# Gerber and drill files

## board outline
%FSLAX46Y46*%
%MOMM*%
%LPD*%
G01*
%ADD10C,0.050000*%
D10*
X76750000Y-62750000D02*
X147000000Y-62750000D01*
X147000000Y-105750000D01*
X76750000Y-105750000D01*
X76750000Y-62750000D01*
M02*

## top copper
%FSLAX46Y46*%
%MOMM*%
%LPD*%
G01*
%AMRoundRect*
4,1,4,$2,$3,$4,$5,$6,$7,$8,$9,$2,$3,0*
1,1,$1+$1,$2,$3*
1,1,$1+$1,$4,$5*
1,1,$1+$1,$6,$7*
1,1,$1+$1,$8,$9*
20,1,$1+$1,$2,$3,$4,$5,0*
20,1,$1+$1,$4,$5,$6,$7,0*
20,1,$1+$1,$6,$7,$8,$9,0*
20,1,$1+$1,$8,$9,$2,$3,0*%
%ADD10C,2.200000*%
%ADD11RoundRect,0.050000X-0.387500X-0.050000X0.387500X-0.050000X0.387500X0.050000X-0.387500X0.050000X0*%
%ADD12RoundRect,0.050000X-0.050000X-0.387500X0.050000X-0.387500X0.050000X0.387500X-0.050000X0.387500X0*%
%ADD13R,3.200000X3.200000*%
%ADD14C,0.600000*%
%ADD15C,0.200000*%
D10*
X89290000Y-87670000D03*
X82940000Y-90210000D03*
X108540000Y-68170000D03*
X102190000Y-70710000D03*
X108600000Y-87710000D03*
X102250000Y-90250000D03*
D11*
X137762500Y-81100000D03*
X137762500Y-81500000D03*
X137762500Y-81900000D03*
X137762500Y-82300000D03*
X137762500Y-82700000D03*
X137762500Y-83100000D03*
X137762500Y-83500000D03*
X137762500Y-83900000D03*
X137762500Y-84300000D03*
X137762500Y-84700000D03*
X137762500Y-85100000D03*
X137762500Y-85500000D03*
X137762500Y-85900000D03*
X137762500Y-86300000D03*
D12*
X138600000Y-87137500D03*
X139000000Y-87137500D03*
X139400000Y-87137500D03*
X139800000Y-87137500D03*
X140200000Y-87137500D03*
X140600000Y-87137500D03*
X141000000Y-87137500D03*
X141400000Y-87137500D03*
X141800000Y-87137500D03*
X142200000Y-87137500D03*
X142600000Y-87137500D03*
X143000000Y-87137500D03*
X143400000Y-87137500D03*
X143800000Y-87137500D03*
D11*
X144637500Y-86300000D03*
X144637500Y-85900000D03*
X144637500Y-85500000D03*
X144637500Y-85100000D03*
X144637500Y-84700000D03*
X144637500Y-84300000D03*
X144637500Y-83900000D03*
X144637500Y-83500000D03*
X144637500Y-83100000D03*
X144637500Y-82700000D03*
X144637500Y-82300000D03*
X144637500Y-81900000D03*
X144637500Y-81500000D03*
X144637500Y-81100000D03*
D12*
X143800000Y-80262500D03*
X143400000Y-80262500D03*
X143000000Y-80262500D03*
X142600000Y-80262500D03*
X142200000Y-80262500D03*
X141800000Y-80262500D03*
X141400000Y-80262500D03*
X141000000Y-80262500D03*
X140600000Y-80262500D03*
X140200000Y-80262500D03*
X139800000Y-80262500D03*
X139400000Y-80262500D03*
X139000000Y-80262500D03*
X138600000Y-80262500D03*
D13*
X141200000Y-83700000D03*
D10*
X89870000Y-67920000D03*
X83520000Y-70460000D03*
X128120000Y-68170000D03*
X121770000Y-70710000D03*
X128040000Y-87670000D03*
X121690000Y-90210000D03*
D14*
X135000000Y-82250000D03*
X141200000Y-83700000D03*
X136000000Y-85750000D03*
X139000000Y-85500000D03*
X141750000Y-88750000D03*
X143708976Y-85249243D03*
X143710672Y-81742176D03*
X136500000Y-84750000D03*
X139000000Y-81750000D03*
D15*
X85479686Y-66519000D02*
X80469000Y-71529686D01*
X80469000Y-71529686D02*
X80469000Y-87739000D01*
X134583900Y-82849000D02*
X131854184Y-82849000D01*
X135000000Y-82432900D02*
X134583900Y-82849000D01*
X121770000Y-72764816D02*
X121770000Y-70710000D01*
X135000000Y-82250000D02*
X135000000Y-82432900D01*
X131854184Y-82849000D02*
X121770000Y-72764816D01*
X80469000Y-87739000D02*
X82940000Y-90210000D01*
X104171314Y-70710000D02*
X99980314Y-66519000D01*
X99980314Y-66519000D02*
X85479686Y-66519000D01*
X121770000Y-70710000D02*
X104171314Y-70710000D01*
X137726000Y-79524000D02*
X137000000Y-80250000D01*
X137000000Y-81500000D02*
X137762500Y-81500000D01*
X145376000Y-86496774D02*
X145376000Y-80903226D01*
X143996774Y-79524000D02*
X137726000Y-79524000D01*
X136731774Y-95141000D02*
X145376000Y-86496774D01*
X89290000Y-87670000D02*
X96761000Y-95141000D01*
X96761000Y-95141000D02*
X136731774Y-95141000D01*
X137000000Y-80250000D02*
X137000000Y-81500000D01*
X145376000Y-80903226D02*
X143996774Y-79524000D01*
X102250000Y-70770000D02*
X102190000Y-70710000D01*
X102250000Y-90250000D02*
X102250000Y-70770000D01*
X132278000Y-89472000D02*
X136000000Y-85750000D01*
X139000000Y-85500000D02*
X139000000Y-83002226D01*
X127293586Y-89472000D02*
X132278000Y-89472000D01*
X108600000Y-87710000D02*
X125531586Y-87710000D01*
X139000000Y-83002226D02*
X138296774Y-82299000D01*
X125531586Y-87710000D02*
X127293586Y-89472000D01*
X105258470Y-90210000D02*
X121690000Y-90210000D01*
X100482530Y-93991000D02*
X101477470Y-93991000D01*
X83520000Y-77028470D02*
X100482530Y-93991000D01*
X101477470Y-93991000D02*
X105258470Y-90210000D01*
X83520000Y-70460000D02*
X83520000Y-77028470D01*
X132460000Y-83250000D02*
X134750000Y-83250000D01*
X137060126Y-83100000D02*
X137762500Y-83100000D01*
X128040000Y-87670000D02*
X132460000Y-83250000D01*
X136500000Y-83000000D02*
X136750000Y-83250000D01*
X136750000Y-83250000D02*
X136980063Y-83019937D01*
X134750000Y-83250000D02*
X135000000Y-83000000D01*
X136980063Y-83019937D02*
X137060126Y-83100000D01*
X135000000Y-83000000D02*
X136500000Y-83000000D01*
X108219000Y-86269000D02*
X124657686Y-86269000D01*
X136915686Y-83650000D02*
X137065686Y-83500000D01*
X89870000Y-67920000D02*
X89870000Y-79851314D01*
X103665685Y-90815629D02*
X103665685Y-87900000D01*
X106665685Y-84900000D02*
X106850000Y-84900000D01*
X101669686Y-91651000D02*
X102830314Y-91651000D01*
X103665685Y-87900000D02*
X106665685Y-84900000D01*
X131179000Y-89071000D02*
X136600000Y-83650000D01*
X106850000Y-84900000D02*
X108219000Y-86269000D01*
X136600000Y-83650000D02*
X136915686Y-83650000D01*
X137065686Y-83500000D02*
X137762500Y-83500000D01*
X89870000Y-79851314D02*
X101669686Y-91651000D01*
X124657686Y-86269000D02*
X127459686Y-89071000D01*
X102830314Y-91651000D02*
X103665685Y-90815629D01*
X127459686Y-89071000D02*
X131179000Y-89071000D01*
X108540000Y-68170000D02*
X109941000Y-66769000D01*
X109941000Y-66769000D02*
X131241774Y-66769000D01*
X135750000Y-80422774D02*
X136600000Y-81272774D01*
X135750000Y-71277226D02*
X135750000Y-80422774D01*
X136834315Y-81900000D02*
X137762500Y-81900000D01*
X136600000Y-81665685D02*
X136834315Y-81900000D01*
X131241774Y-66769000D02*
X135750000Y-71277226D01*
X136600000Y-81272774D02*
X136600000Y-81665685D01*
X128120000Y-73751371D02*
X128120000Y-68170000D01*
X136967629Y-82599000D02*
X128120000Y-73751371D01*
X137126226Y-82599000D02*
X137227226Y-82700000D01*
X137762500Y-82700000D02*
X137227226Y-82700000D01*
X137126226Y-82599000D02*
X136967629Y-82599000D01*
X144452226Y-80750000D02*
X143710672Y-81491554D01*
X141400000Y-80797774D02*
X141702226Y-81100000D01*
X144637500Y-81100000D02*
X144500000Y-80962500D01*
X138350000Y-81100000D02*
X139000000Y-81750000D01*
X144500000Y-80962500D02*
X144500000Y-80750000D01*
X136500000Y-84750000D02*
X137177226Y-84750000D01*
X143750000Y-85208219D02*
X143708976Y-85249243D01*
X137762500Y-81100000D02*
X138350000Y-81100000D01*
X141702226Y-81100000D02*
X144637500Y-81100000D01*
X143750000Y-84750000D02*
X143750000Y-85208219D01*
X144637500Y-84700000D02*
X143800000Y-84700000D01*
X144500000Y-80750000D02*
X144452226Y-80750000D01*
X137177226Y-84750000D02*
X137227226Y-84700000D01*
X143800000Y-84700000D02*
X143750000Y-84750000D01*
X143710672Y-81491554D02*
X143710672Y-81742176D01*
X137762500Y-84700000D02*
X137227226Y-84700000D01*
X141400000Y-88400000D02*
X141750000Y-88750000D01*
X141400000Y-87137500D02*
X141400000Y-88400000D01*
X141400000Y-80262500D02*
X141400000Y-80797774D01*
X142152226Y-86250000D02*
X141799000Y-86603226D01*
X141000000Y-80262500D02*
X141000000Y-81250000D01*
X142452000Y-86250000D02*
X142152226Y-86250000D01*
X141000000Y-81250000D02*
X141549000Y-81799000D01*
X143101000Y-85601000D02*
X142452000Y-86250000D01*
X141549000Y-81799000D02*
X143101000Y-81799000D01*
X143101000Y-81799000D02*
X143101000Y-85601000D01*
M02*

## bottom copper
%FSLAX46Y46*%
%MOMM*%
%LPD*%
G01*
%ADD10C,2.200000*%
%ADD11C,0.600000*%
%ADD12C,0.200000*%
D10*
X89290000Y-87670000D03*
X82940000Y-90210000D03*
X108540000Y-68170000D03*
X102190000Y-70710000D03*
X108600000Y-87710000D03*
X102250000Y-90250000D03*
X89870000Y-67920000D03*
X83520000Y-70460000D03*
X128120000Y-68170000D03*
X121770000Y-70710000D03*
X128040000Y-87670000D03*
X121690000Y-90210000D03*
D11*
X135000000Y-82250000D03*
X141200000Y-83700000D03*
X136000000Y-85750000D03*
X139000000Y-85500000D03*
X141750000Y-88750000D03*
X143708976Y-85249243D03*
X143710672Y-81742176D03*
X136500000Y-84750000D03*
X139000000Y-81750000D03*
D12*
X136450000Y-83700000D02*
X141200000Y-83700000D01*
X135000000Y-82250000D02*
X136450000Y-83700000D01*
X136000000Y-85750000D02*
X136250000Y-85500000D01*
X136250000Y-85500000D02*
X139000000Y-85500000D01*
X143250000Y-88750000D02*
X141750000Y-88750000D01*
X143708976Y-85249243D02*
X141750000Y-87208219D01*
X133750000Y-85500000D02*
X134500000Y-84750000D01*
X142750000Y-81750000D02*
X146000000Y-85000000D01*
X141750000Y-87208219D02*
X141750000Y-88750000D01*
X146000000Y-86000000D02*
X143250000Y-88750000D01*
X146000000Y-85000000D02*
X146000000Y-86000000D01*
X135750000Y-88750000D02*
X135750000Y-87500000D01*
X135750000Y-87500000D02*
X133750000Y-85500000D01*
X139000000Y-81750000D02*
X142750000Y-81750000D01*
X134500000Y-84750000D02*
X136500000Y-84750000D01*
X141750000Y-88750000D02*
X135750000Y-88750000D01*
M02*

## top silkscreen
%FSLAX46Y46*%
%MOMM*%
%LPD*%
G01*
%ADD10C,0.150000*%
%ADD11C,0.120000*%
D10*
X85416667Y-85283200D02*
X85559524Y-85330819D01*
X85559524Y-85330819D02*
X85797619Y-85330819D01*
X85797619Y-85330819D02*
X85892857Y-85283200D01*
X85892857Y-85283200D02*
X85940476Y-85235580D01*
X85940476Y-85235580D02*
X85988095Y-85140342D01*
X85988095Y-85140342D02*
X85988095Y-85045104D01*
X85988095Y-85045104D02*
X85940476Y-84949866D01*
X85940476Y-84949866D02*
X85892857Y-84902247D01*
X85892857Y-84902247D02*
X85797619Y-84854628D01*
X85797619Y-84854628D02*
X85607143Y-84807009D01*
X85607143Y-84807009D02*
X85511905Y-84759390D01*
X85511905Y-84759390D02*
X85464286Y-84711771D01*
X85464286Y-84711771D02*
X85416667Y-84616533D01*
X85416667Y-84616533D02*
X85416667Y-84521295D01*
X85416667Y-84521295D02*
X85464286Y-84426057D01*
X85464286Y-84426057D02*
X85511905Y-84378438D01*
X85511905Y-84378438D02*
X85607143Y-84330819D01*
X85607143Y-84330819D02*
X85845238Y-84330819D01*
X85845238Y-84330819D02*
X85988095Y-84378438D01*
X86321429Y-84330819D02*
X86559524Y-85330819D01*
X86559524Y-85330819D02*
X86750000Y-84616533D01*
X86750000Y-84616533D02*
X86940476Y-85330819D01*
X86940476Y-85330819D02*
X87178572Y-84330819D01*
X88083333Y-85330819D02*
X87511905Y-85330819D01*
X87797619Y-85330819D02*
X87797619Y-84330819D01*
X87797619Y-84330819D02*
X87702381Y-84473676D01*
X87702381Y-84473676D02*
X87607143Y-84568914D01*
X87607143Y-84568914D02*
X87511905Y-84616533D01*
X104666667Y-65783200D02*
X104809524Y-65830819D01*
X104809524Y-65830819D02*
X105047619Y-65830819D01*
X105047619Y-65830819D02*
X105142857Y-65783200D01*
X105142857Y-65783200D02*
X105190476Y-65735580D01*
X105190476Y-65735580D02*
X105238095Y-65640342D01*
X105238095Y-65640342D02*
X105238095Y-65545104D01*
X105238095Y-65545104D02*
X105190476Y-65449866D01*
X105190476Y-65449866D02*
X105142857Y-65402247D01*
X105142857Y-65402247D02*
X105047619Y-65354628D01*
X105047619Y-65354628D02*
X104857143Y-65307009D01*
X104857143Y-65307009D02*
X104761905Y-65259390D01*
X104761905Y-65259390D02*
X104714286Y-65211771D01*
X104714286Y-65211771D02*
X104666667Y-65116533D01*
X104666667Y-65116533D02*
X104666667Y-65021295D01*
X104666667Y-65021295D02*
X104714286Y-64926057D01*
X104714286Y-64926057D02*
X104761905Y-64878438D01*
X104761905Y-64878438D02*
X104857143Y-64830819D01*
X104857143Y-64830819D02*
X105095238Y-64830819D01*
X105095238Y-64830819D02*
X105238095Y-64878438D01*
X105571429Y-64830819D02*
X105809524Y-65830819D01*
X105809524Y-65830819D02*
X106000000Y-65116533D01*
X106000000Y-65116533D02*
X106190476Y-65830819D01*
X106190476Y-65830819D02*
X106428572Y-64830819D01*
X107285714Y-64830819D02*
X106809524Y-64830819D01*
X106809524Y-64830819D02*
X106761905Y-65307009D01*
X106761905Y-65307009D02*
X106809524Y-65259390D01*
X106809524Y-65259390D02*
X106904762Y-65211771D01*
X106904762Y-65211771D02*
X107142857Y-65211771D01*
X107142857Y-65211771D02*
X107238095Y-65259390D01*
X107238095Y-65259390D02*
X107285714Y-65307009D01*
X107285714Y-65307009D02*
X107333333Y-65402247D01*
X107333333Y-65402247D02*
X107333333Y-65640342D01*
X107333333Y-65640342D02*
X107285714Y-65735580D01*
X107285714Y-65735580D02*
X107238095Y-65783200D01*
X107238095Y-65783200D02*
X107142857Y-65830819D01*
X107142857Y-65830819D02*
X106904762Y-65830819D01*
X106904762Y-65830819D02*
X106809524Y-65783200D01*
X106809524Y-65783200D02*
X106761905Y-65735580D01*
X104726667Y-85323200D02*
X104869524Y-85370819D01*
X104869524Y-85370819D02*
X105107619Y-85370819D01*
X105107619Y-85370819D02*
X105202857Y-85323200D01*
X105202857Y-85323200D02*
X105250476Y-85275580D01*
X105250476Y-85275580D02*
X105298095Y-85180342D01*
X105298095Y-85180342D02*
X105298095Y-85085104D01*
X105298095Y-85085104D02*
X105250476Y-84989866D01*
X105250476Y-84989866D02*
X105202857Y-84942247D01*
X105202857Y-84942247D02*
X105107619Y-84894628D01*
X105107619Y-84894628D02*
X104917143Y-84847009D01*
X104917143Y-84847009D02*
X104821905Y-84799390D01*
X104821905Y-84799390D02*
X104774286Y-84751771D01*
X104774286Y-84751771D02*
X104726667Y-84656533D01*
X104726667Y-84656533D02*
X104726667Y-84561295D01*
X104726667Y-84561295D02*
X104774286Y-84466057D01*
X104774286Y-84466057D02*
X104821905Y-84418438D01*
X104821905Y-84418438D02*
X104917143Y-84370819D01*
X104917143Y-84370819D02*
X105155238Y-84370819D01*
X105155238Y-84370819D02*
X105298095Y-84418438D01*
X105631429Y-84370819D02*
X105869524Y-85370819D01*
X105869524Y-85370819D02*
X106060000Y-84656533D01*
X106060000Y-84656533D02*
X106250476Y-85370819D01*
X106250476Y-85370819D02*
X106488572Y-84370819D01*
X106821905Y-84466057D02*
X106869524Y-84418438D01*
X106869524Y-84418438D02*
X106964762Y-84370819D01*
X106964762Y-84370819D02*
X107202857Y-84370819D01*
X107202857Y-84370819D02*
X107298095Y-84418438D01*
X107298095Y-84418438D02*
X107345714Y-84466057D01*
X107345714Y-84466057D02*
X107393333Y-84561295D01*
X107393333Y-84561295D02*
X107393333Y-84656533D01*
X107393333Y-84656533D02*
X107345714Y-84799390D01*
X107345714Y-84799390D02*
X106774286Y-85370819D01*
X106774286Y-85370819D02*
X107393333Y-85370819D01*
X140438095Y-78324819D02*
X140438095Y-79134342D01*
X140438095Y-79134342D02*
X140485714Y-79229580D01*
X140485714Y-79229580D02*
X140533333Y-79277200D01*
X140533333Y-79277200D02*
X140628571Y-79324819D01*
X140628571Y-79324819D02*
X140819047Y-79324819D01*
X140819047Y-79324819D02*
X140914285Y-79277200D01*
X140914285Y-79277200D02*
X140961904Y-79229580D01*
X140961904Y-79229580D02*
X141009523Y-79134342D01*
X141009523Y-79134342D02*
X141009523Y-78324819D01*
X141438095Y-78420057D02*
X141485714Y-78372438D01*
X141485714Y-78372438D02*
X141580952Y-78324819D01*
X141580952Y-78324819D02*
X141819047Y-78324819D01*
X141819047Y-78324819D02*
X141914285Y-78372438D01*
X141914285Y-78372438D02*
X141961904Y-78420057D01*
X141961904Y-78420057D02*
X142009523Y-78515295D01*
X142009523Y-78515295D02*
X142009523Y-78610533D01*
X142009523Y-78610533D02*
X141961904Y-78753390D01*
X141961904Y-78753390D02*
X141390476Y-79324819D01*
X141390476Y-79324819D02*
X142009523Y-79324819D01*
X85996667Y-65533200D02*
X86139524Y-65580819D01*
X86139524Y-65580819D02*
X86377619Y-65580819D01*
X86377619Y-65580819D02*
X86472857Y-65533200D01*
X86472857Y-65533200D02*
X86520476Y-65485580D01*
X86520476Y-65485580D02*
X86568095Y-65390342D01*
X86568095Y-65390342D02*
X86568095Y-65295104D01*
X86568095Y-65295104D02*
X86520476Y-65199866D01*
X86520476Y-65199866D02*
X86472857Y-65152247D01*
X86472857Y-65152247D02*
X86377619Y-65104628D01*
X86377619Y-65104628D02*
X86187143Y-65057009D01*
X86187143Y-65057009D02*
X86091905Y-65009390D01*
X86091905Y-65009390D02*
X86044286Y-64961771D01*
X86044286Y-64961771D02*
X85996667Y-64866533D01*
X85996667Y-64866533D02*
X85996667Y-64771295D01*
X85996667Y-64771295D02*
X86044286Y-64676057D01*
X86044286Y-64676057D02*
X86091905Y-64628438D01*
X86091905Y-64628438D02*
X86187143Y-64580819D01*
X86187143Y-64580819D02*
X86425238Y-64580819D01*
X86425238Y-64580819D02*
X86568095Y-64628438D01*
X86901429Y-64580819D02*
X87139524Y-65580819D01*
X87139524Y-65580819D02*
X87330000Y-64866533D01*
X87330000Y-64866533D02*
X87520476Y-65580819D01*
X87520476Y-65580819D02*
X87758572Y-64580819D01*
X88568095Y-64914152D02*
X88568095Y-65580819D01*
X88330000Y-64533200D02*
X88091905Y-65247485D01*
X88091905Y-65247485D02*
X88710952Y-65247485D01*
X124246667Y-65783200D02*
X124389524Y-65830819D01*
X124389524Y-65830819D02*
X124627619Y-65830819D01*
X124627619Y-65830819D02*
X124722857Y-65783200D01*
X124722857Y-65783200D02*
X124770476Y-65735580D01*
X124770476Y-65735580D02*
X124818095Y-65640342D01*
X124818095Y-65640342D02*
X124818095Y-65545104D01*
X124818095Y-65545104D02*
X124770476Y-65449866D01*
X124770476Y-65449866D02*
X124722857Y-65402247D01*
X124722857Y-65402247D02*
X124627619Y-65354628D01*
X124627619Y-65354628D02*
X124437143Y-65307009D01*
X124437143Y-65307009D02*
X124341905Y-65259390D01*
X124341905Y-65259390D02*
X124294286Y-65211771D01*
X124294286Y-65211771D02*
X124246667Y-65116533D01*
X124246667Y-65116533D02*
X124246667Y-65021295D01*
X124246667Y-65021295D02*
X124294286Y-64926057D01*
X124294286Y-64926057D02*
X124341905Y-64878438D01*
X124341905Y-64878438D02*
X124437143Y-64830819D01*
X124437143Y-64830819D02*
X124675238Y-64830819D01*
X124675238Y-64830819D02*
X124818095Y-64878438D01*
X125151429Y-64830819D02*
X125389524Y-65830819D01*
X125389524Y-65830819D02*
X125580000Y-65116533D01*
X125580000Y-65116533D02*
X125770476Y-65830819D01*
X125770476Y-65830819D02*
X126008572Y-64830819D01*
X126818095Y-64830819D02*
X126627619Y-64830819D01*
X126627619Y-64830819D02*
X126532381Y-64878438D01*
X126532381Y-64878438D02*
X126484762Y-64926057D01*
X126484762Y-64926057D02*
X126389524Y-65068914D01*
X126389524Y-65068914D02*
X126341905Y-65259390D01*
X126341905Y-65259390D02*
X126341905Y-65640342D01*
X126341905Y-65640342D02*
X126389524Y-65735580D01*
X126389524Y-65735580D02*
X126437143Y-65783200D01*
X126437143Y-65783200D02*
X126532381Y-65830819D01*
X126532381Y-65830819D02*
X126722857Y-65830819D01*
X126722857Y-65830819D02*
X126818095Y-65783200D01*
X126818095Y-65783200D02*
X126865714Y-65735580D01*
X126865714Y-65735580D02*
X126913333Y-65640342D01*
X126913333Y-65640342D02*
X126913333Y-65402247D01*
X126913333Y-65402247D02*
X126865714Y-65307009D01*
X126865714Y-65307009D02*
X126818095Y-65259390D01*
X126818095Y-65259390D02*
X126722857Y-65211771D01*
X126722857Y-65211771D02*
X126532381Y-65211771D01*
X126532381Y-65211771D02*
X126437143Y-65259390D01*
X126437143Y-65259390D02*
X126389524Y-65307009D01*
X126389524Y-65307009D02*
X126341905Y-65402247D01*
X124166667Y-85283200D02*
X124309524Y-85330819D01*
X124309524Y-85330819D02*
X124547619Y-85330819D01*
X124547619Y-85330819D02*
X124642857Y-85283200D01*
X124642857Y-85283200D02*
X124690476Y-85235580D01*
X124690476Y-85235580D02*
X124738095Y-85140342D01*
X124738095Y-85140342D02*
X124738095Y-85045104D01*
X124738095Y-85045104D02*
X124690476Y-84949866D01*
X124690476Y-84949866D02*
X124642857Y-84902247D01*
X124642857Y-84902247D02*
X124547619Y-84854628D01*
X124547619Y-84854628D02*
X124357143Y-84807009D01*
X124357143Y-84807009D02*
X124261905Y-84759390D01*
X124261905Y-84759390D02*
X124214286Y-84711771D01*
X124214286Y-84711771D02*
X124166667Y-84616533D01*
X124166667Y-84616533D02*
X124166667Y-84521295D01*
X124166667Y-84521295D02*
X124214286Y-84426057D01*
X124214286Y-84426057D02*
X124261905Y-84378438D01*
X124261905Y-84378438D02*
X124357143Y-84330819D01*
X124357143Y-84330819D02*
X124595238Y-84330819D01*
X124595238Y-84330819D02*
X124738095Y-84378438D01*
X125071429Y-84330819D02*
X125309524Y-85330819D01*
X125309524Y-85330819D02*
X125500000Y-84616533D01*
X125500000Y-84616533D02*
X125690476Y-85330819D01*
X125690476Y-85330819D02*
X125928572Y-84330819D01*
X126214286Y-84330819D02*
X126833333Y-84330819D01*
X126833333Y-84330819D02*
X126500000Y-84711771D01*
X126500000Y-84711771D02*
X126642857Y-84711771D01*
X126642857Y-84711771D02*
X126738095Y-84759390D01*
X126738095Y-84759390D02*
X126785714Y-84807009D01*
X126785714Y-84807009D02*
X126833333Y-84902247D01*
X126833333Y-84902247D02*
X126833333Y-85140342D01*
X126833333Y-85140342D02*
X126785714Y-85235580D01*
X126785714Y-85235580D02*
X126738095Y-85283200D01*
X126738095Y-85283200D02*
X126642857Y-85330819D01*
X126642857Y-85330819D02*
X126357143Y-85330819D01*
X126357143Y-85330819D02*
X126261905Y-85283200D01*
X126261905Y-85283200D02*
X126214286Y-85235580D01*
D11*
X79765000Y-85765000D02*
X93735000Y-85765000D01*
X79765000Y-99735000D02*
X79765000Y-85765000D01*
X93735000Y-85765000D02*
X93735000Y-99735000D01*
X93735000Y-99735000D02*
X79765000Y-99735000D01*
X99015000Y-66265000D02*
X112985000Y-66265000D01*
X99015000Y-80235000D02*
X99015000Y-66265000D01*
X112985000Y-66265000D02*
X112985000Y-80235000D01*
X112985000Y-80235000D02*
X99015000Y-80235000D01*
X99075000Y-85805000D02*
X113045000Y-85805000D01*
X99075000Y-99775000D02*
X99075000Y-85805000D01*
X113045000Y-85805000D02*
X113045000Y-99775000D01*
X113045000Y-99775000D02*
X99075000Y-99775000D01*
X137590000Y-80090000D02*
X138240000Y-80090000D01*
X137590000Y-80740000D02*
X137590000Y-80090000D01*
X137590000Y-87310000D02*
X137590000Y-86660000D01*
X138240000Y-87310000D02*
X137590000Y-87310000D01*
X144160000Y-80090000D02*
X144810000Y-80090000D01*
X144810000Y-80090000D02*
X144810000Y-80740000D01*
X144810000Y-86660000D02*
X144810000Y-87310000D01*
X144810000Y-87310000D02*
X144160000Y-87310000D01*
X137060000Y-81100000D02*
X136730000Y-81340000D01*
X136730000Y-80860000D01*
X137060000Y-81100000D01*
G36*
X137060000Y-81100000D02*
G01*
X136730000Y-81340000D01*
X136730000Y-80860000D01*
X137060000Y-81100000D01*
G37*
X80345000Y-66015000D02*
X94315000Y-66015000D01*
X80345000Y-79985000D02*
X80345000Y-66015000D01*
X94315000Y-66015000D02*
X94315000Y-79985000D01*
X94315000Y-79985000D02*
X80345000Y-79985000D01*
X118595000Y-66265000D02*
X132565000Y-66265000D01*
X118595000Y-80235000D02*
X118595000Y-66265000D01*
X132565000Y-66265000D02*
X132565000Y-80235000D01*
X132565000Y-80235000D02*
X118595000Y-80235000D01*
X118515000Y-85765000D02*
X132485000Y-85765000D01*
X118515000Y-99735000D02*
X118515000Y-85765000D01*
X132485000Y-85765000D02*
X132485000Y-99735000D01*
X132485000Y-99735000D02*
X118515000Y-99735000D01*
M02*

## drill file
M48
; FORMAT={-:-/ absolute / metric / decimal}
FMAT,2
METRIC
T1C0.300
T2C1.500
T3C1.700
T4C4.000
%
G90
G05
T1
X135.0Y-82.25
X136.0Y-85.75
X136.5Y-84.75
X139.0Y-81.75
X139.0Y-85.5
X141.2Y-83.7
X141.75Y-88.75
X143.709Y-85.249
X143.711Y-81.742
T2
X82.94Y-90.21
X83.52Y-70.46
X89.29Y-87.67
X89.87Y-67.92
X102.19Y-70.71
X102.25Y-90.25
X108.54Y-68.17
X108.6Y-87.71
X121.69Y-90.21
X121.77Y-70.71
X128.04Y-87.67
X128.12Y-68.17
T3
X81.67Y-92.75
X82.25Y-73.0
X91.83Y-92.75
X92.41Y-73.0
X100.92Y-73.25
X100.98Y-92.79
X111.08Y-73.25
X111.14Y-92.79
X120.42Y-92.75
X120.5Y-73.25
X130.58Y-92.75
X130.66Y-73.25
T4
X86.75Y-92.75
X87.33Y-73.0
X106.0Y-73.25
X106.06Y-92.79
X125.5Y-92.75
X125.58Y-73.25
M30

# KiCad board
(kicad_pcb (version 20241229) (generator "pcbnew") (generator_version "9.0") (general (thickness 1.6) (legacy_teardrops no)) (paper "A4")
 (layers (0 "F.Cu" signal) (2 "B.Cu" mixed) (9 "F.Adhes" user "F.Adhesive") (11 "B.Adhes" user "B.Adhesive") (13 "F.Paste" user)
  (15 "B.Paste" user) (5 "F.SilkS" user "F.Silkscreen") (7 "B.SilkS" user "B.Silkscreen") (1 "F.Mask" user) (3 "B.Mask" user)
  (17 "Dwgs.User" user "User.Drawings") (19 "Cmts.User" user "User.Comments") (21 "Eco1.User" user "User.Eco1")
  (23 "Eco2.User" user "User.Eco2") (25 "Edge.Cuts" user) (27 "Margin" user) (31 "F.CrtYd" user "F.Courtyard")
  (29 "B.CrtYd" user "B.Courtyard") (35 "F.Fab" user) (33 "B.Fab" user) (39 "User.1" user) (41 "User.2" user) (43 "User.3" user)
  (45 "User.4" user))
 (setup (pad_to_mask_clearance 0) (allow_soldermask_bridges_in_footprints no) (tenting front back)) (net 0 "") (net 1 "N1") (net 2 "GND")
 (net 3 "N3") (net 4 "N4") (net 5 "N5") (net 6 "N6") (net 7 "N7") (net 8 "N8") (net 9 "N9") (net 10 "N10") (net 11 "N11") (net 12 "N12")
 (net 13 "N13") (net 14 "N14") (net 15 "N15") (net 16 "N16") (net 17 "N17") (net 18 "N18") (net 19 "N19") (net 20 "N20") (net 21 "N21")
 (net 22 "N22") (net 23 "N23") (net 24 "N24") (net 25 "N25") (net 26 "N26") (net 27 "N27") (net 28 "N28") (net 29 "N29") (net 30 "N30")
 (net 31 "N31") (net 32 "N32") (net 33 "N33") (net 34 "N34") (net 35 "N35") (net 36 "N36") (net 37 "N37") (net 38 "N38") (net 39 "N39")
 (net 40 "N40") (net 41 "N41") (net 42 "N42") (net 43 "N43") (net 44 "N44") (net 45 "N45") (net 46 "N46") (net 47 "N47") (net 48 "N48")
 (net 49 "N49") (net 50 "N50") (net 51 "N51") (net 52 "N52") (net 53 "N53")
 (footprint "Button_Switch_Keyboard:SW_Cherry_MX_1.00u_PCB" (layer "F.Cu") (at 89.29 87.67)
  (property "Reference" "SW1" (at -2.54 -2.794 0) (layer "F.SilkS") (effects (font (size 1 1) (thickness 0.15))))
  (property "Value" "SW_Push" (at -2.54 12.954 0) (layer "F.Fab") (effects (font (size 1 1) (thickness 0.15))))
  (fp_line (start -9.525 -1.905) (end 4.445 -1.905) (stroke (width 0.12) (type solid)) (layer "F.SilkS"))
  (fp_line (start -9.525 12.065) (end -9.525 -1.905) (stroke (width 0.12) (type solid)) (layer "F.SilkS"))
  (fp_line (start 4.445 -1.905) (end 4.445 12.065) (stroke (width 0.12) (type solid)) (layer "F.SilkS"))
  (fp_line (start 4.445 12.065) (end -9.525 12.065) (stroke (width 0.12) (type solid)) (layer "F.SilkS"))
  (pad "" np_thru_hole circle (at -7.62 5.08) (size 1.7 1.7) (drill 1.7) (layers "*.Cu" "*.Mask"))
  (pad "" np_thru_hole circle (at -2.54 5.08) (size 4 4) (drill 4) (layers "*.Cu" "*.Mask"))
  (pad "" np_thru_hole circle (at 2.54 5.08) (size 1.7 1.7) (drill 1.7) (layers "*.Cu" "*.Mask"))
  (pad "1" thru_hole circle (at 0 0) (size 2.2 2.2) (drill 1.5) (layers "*.Cu" "*.Mask") (remove_unused_layers no) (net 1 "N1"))
  (pad "2" thru_hole circle (at -6.35 2.54) (size 2.2 2.2) (drill 1.5) (layers "*.Cu" "*.Mask") (remove_unused_layers no) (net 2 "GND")))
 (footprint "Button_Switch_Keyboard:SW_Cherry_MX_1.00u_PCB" (layer "F.Cu") (at 108.54 68.17)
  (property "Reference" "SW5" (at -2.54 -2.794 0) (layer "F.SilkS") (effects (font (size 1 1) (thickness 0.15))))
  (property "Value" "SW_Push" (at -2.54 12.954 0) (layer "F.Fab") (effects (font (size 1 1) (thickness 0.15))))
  (fp_line (start -9.525 -1.905) (end 4.445 -1.905) (stroke (width 0.12) (type solid)) (layer "F.SilkS"))
  (fp_line (start -9.525 12.065) (end -9.525 -1.905) (stroke (width 0.12) (type solid)) (layer "F.SilkS"))
  (fp_line (start 4.445 -1.905) (end 4.445 12.065) (stroke (width 0.12) (type solid)) (layer "F.SilkS"))
  (fp_line (start 4.445 12.065) (end -9.525 12.065) (stroke (width 0.12) (type solid)) (layer "F.SilkS"))
  (pad "" np_thru_hole circle (at -7.62 5.08) (size 1.7 1.7) (drill 1.7) (layers "*.Cu" "*.Mask"))
  (pad "" np_thru_hole circle (at -2.54 5.08) (size 4 4) (drill 4) (layers "*.Cu" "*.Mask"))
  (pad "" np_thru_hole circle (at 2.54 5.08) (size 1.7 1.7) (drill 1.7) (layers "*.Cu" "*.Mask"))
  (pad "1" thru_hole circle (at 0 0) (size 2.2 2.2) (drill 1.5) (layers "*.Cu" "*.Mask") (remove_unused_layers no) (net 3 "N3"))
  (pad "2" thru_hole circle (at -6.35 2.54) (size 2.2 2.2) (drill 1.5) (layers "*.Cu" "*.Mask") (remove_unused_layers no) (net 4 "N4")))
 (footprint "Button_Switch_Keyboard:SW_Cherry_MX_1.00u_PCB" (layer "F.Cu") (at 108.6 87.71)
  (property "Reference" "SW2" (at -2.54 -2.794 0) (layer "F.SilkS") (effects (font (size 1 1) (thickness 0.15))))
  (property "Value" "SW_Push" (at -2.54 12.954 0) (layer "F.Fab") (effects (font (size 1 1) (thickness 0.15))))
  (fp_line (start -9.525 -1.905) (end 4.445 -1.905) (stroke (width 0.12) (type solid)) (layer "F.SilkS"))
  (fp_line (start -9.525 12.065) (end -9.525 -1.905) (stroke (width 0.12) (type solid)) (layer "F.SilkS"))
  (fp_line (start 4.445 -1.905) (end 4.445 12.065) (stroke (width 0.12) (type solid)) (layer "F.SilkS"))
  (fp_line (start 4.445 12.065) (end -9.525 12.065) (stroke (width 0.12) (type solid)) (layer "F.SilkS"))
  (pad "" np_thru_hole circle (at -7.62 5.08) (size 1.7 1.7) (drill 1.7) (layers "*.Cu" "*.Mask"))
  (pad "" np_thru_hole circle (at -2.54 5.08) (size 4 4) (drill 4) (layers "*.Cu" "*.Mask"))
  (pad "" np_thru_hole circle (at 2.54 5.08) (size 1.7 1.7) (drill 1.7) (layers "*.Cu" "*.Mask"))
  (pad "1" thru_hole circle (at 0 0) (size 2.2 2.2) (drill 1.5) (layers "*.Cu" "*.Mask") (remove_unused_layers no) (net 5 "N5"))
  (pad "2" thru_hole circle (at -6.35 2.54) (size 2.2 2.2) (drill 1.5) (layers "*.Cu" "*.Mask") (remove_unused_layers no) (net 4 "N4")))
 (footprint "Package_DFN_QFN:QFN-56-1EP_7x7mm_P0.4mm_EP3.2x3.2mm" (layer "F.Cu") (at 141.2 83.7)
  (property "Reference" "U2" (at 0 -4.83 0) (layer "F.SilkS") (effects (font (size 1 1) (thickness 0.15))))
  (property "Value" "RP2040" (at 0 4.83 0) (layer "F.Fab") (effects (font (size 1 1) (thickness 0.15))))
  (fp_line (start -3.61 -3.61) (end -2.96 -3.61) (stroke (width 0.12) (type solid)) (layer "F.SilkS"))
  (fp_line (start -3.61 -2.96) (end -3.61 -3.61) (stroke (width 0.12) (type solid)) (layer "F.SilkS"))
  (fp_line (start -3.61 3.61) (end -3.61 2.96) (stroke (width 0.12) (type solid)) (layer "F.SilkS"))
  (fp_line (start -2.96 3.61) (end -3.61 3.61) (stroke (width 0.12) (type solid)) (layer "F.SilkS"))
  (fp_line (start 2.96 -3.61) (end 3.61 -3.61) (stroke (width 0.12) (type solid)) (layer "F.SilkS"))
  (fp_line (start 3.61 -3.61) (end 3.61 -2.96) (stroke (width 0.12) (type solid)) (layer "F.SilkS"))
  (fp_line (start 3.61 2.96) (end 3.61 3.61) (stroke (width 0.12) (type solid)) (layer "F.SilkS"))
  (fp_line (start 3.61 3.61) (end 2.96 3.61) (stroke (width 0.12) (type solid)) (layer "F.SilkS"))
  (fp_poly (pts (xy -4.14 -2.6) (xy -4.47 -2.36) (xy -4.47 -2.84)) (stroke (width 0.12) (type solid)) (fill yes) (layer "F.SilkS"))
  (pad "" smd roundrect (at -0.8 -0.8) (size 1.29 1.29) (layers "F.Paste") (roundrect_rratio 0.193798))
  (pad "" smd roundrect (at -0.8 0.8) (size 1.29 1.29) (layers "F.Paste") (roundrect_rratio 0.193798))
  (pad "" smd roundrect (at 0.8 -0.8) (size 1.29 1.29) (layers "F.Paste") (roundrect_rratio 0.193798))
  (pad "" smd roundrect (at 0.8 0.8) (size 1.29 1.29) (layers "F.Paste") (roundrect_rratio 0.193798))
  (pad "1" smd roundrect (at -3.4375 -2.6) (size 0.875 0.2) (layers "F.Cu" "F.Mask" "F.Paste") (roundrect_rratio 0.25) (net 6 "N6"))
  (pad "2" smd roundrect (at -3.4375 -2.2) (size 0.875 0.2) (layers "F.Cu" "F.Mask" "F.Paste") (roundrect_rratio 0.25) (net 1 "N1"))
  (pad "3" smd roundrect (at -3.4375 -1.8) (size 0.875 0.2) (layers "F.Cu" "F.Mask" "F.Paste") (roundrect_rratio 0.25) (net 3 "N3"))
  (pad "4" smd roundrect (at -3.4375 -1.4) (size 0.875 0.2) (layers "F.Cu" "F.Mask" "F.Paste") (roundrect_rratio 0.25) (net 5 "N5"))
  (pad "5" smd roundrect (at -3.4375 -1) (size 0.875 0.2) (layers "F.Cu" "F.Mask" "F.Paste") (roundrect_rratio 0.25) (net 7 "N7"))
  (pad "6" smd roundrect (at -3.4375 -0.6) (size 0.875 0.2) (layers "F.Cu" "F.Mask" "F.Paste") (roundrect_rratio 0.25) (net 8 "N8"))
  (pad "7" smd roundrect (at -3.4375 -0.2) (size 0.875 0.2) (layers "F.Cu" "F.Mask" "F.Paste") (roundrect_rratio 0.25) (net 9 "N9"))
  (pad "8" smd roundrect (at -3.4375 0.2) (size 0.875 0.2) (layers "F.Cu" "F.Mask" "F.Paste") (roundrect_rratio 0.25) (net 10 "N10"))
  (pad "9" smd roundrect (at -3.4375 0.6) (size 0.875 0.2) (layers "F.Cu" "F.Mask" "F.Paste") (roundrect_rratio 0.25) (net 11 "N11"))
  (pad "10" smd roundrect (at -3.4375 1) (size 0.875 0.2) (layers "F.Cu" "F.Mask" "F.Paste") (roundrect_rratio 0.25) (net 6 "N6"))
  (pad "11" smd roundrect (at -3.4375 1.4) (size 0.875 0.2) (layers "F.Cu" "F.Mask" "F.Paste") (roundrect_rratio 0.25) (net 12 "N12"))
  (pad "12" smd roundrect (at -3.4375 1.8) (size 0.875 0.2) (layers "F.Cu" "F.Mask" "F.Paste") (roundrect_rratio 0.25) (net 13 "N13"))
  (pad "13" smd roundrect (at -3.4375 2.2) (size 0.875 0.2) (layers "F.Cu" "F.Mask" "F.Paste") (roundrect_rratio 0.25) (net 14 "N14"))
  (pad "14" smd roundrect (at -3.4375 2.6) (size 0.875 0.2) (layers "F.Cu" "F.Mask" "F.Paste") (roundrect_rratio 0.25) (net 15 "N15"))
  (pad "15" smd roundrect (at -2.6 3.4375) (size 0.2 0.875) (layers "F.Cu" "F.Mask" "F.Paste") (roundrect_rratio 0.25) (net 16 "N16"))
  (pad "16" smd roundrect (at -2.2 3.4375) (size 0.2 0.875) (layers "F.Cu" "F.Mask" "F.Paste") (roundrect_rratio 0.25) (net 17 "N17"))
  (pad "17" smd roundrect (at -1.8 3.4375) (size 0.2 0.875) (layers "F.Cu" "F.Mask" "F.Paste") (roundrect_rratio 0.25) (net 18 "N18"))
  (pad "18" smd roundrect (at -1.4 3.4375) (size 0.2 0.875) (layers "F.Cu" "F.Mask" "F.Paste") (roundrect_rratio 0.25) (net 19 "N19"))
  (pad "19" smd roundrect (at -1 3.4375) (size 0.2 0.875) (layers "F.Cu" "F.Mask" "F.Paste") (roundrect_rratio 0.25) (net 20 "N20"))
  (pad "20" smd roundrect (at -0.6 3.4375) (size 0.2 0.875) (layers "F.Cu" "F.Mask" "F.Paste") (roundrect_rratio 0.25) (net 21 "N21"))
  (pad "21" smd roundrect (at -0.2 3.4375) (size 0.2 0.875) (layers "F.Cu" "F.Mask" "F.Paste") (roundrect_rratio 0.25) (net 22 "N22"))
  (pad "22" smd roundrect (at 0.2 3.4375) (size 0.2 0.875) (layers "F.Cu" "F.Mask" "F.Paste") (roundrect_rratio 0.25) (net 6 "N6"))
  (pad "23" smd roundrect (at 0.6 3.4375) (size 0.2 0.875) (layers "F.Cu" "F.Mask" "F.Paste") (roundrect_rratio 0.25) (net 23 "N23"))
  (pad "24" smd roundrect (at 1 3.4375) (size 0.2 0.875) (layers "F.Cu" "F.Mask" "F.Paste") (roundrect_rratio 0.25) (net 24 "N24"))
  (pad "25" smd roundrect (at 1.4 3.4375) (size 0.2 0.875) (layers "F.Cu" "F.Mask" "F.Paste") (roundrect_rratio 0.25) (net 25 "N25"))
  (pad "26" smd roundrect (at 1.8 3.4375) (size 0.2 0.875) (layers "F.Cu" "F.Mask" "F.Paste") (roundrect_rratio 0.25) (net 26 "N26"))
  (pad "27" smd roundrect (at 2.2 3.4375) (size 0.2 0.875) (layers "F.Cu" "F.Mask" "F.Paste") (roundrect_rratio 0.25) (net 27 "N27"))
  (pad "28" smd roundrect (at 2.6 3.4375) (size 0.2 0.875) (layers "F.Cu" "F.Mask" "F.Paste") (roundrect_rratio 0.25) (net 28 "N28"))
  (pad "29" smd roundrect (at 3.4375 2.6) (size 0.875 0.2) (layers "F.Cu" "F.Mask" "F.Paste") (roundrect_rratio 0.25) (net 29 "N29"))
  (pad "30" smd roundrect (at 3.4375 2.2) (size 0.875 0.2) (layers "F.Cu" "F.Mask" "F.Paste") (roundrect_rratio 0.25) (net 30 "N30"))
  (pad "31" smd roundrect (at 3.4375 1.8) (size 0.875 0.2) (layers "F.Cu" "F.Mask" "F.Paste") (roundrect_rratio 0.25) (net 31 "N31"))
  (pad "32" smd roundrect (at 3.4375 1.4) (size 0.875 0.2) (layers "F.Cu" "F.Mask" "F.Paste") (roundrect_rratio 0.25) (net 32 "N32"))
  (pad "33" smd roundrect (at 3.4375 1) (size 0.875 0.2) (layers "F.Cu" "F.Mask" "F.Paste") (roundrect_rratio 0.25) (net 6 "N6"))
  (pad "34" smd roundrect (at 3.4375 0.6) (size 0.875 0.2) (layers "F.Cu" "F.Mask" "F.Paste") (roundrect_rratio 0.25) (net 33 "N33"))
  (pad "35" smd roundrect (at 3.4375 0.2) (size 0.875 0.2) (layers "F.Cu" "F.Mask" "F.Paste") (roundrect_rratio 0.25) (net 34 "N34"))
  (pad "36" smd roundrect (at 3.4375 -0.2) (size 0.875 0.2) (layers "F.Cu" "F.Mask" "F.Paste") (roundrect_rratio 0.25) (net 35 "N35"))
  (pad "37" smd roundrect (at 3.4375 -0.6) (size 0.875 0.2) (layers "F.Cu" "F.Mask" "F.Paste") (roundrect_rratio 0.25) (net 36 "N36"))
  (pad "38" smd roundrect (at 3.4375 -1) (size 0.875 0.2) (layers "F.Cu" "F.Mask" "F.Paste") (roundrect_rratio 0.25) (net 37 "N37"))
  (pad "39" smd roundrect (at 3.4375 -1.4) (size 0.875 0.2) (layers "F.Cu" "F.Mask" "F.Paste") (roundrect_rratio 0.25) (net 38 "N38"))
  (pad "40" smd roundrect (at 3.4375 -1.8) (size 0.875 0.2) (layers "F.Cu" "F.Mask" "F.Paste") (roundrect_rratio 0.25) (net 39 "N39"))
  (pad "41" smd roundrect (at 3.4375 -2.2) (size 0.875 0.2) (layers "F.Cu" "F.Mask" "F.Paste") (roundrect_rratio 0.25) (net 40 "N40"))
  (pad "42" smd roundrect (at 3.4375 -2.6) (size 0.875 0.2) (layers "F.Cu" "F.Mask" "F.Paste") (roundrect_rratio 0.25) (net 6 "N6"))
  (pad "43" smd roundrect (at 2.6 -3.4375) (size 0.2 0.875) (layers "F.Cu" "F.Mask" "F.Paste") (roundrect_rratio 0.25) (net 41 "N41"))
  (pad "44" smd roundrect (at 2.2 -3.4375) (size 0.2 0.875) (layers "F.Cu" "F.Mask" "F.Paste") (roundrect_rratio 0.25) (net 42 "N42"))
  (pad "45" smd roundrect (at 1.8 -3.4375) (size 0.2 0.875) (layers "F.Cu" "F.Mask" "F.Paste") (roundrect_rratio 0.25) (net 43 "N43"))
  (pad "46" smd roundrect (at 1.4 -3.4375) (size 0.2 0.875) (layers "F.Cu" "F.Mask" "F.Paste") (roundrect_rratio 0.25) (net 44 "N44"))
  (pad "47" smd roundrect (at 1 -3.4375) (size 0.2 0.875) (layers "F.Cu" "F.Mask" "F.Paste") (roundrect_rratio 0.25) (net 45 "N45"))
  (pad "48" smd roundrect (at 0.6 -3.4375) (size 0.2 0.875) (layers "F.Cu" "F.Mask" "F.Paste") (roundrect_rratio 0.25) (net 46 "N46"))
  (pad "49" smd roundrect (at 0.2 -3.4375) (size 0.2 0.875) (layers "F.Cu" "F.Mask" "F.Paste") (roundrect_rratio 0.25) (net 6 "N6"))
  (pad "50" smd roundrect (at -0.2 -3.4375) (size 0.2 0.875) (layers "F.Cu" "F.Mask" "F.Paste") (roundrect_rratio 0.25) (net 23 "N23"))
  (pad "51" smd roundrect (at -0.6 -3.4375) (size 0.2 0.875) (layers "F.Cu" "F.Mask" "F.Paste") (roundrect_rratio 0.25) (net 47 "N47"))
  (pad "52" smd roundrect (at -1 -3.4375) (size 0.2 0.875) (layers "F.Cu" "F.Mask" "F.Paste") (roundrect_rratio 0.25) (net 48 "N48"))
  (pad "53" smd roundrect (at -1.4 -3.4375) (size 0.2 0.875) (layers "F.Cu" "F.Mask" "F.Paste") (roundrect_rratio 0.25) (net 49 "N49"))
  (pad "54" smd roundrect (at -1.8 -3.4375) (size 0.2 0.875) (layers "F.Cu" "F.Mask" "F.Paste") (roundrect_rratio 0.25) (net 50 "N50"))
  (pad "55" smd roundrect (at -2.2 -3.4375) (size 0.2 0.875) (layers "F.Cu" "F.Mask" "F.Paste") (roundrect_rratio 0.25) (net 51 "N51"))
  (pad "56" smd roundrect (at -2.6 -3.4375) (size 0.2 0.875) (layers "F.Cu" "F.Mask" "F.Paste") (roundrect_rratio 0.25) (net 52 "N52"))
  (pad "57" smd rect (at 0 0) (size 3.2 3.2) (layers "F.Cu" "F.Mask") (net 2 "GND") (zone_connect 2)))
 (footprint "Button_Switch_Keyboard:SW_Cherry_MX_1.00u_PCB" (layer "F.Cu") (at 89.87 67.92)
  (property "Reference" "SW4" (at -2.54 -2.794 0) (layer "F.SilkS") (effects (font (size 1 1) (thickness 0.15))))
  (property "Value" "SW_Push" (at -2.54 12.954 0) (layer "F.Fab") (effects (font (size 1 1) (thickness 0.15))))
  (fp_line (start -9.525 -1.905) (end 4.445 -1.905) (stroke (width 0.12) (type solid)) (layer "F.SilkS"))
  (fp_line (start -9.525 12.065) (end -9.525 -1.905) (stroke (width 0.12) (type solid)) (layer "F.SilkS"))
  (fp_line (start 4.445 -1.905) (end 4.445 12.065) (stroke (width 0.12) (type solid)) (layer "F.SilkS"))
  (fp_line (start 4.445 12.065) (end -9.525 12.065) (stroke (width 0.12) (type solid)) (layer "F.SilkS"))
  (pad "" np_thru_hole circle (at -7.62 5.08) (size 1.7 1.7) (drill 1.7) (layers "*.Cu" "*.Mask"))
  (pad "" np_thru_hole circle (at -2.54 5.08) (size 4 4) (drill 4) (layers "*.Cu" "*.Mask"))
  (pad "" np_thru_hole circle (at 2.54 5.08) (size 1.7 1.7) (drill 1.7) (layers "*.Cu" "*.Mask"))
  (pad "1" thru_hole circle (at 0 0) (size 2.2 2.2) (drill 1.5) (layers "*.Cu" "*.Mask") (remove_unused_layers no) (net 9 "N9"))
  (pad "2" thru_hole circle (at -6.35 2.54) (size 2.2 2.2) (drill 1.5) (layers "*.Cu" "*.Mask") (remove_unused_layers no) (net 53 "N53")))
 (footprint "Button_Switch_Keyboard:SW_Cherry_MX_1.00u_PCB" (layer "F.Cu") (at 128.12 68.17)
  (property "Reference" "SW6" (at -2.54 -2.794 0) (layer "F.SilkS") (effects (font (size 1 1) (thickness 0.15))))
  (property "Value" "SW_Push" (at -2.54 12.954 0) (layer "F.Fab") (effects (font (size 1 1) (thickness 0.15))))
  (fp_line (start -9.525 -1.905) (end 4.445 -1.905) (stroke (width 0.12) (type solid)) (layer "F.SilkS"))
  (fp_line (start -9.525 12.065) (end -9.525 -1.905) (stroke (width 0.12) (type solid)) (layer "F.SilkS"))
  (fp_line (start 4.445 -1.905) (end 4.445 12.065) (stroke (width 0.12) (type solid)) (layer "F.SilkS"))
  (fp_line (start 4.445 12.065) (end -9.525 12.065) (stroke (width 0.12) (type solid)) (layer "F.SilkS"))
  (pad "" np_thru_hole circle (at -7.62 5.08) (size 1.7 1.7) (drill 1.7) (layers "*.Cu" "*.Mask"))
  (pad "" np_thru_hole circle (at -2.54 5.08) (size 4 4) (drill 4) (layers "*.Cu" "*.Mask"))
  (pad "" np_thru_hole circle (at 2.54 5.08) (size 1.7 1.7) (drill 1.7) (layers "*.Cu" "*.Mask"))
  (pad "1" thru_hole circle (at 0 0) (size 2.2 2.2) (drill 1.5) (layers "*.Cu" "*.Mask") (remove_unused_layers no) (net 7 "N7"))
  (pad "2" thru_hole circle (at -6.35 2.54) (size 2.2 2.2) (drill 1.5) (layers "*.Cu" "*.Mask") (remove_unused_layers no) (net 2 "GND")))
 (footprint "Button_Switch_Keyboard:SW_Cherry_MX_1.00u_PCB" (layer "F.Cu") (at 128.04 87.67)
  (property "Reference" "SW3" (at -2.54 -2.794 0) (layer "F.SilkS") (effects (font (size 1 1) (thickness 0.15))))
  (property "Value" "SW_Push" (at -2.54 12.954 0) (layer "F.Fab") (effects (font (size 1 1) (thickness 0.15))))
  (fp_line (start -9.525 -1.905) (end 4.445 -1.905) (stroke (width 0.12) (type solid)) (layer "F.SilkS"))
  (fp_line (start -9.525 12.065) (end -9.525 -1.905) (stroke (width 0.12) (type solid)) (layer "F.SilkS"))
  (fp_line (start 4.445 -1.905) (end 4.445 12.065) (stroke (width 0.12) (type solid)) (layer "F.SilkS"))
  (fp_line (start 4.445 12.065) (end -9.525 12.065) (stroke (width 0.12) (type solid)) (layer "F.SilkS"))
  (pad "" np_thru_hole circle (at -7.62 5.08) (size 1.7 1.7) (drill 1.7) (layers "*.Cu" "*.Mask"))
  (pad "" np_thru_hole circle (at -2.54 5.08) (size 4 4) (drill 4) (layers "*.Cu" "*.Mask"))
  (pad "" np_thru_hole circle (at 2.54 5.08) (size 1.7 1.7) (drill 1.7) (layers "*.Cu" "*.Mask"))
  (pad "1" thru_hole circle (at 0 0) (size 2.2 2.2) (drill 1.5) (layers "*.Cu" "*.Mask") (remove_unused_layers no) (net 8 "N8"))
  (pad "2" thru_hole circle (at -6.35 2.54) (size 2.2 2.2) (drill 1.5) (layers "*.Cu" "*.Mask") (remove_unused_layers no) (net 53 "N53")))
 (gr_rect (start 76.75 62.75) (end 147 105.75) (stroke (width 0.05) (type default)) (fill no) (layer "Edge.Cuts"))
 (segment (start 85.479686 66.519) (end 80.469 71.529686) (width 0.2) (layer "F.Cu") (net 2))
 (segment (start 80.469 71.529686) (end 80.469 87.739) (width 0.2) (layer "F.Cu") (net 2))
 (segment (start 134.5839 82.849) (end 131.854184 82.849) (width 0.2) (layer "F.Cu") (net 2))
 (segment (start 135 82.4329) (end 134.5839 82.849) (width 0.2) (layer "F.Cu") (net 2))
 (segment (start 121.77 72.764816) (end 121.77 70.71) (width 0.2) (layer "F.Cu") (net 2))
 (segment (start 135 82.25) (end 135 82.4329) (width 0.2) (layer "F.Cu") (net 2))
 (segment (start 131.854184 82.849) (end 121.77 72.764816) (width 0.2) (layer "F.Cu") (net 2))
 (segment (start 80.469 87.739) (end 82.94 90.21) (width 0.2) (layer "F.Cu") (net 2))
 (segment (start 104.171314 70.71) (end 99.980314 66.519) (width 0.2) (layer "F.Cu") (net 2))
 (segment (start 99.980314 66.519) (end 85.479686 66.519) (width 0.2) (layer "F.Cu") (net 2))
 (segment (start 121.77 70.71) (end 104.171314 70.71) (width 0.2) (layer "F.Cu") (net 2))
 (via (at 135 82.25) (size 0.6) (drill 0.3) (layers "F.Cu" "B.Cu") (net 2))
 (via (at 141.2 83.7) (size 0.6) (drill 0.3) (layers "F.Cu" "B.Cu") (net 2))
 (segment (start 136.45 83.7) (end 141.2 83.7) (width 0.2) (layer "B.Cu") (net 2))
 (segment (start 135 82.25) (end 136.45 83.7) (width 0.2) (layer "B.Cu") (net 2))
 (segment (start 137.726 79.524) (end 137 80.25) (width 0.2) (layer "F.Cu") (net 1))
 (segment (start 137 81.5) (end 137.7625 81.5) (width 0.2) (layer "F.Cu") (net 1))
 (segment (start 145.376 86.496774) (end 145.376 80.903226) (width 0.2) (layer "F.Cu") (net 1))
 (segment (start 143.996774 79.524) (end 137.726 79.524) (width 0.2) (layer "F.Cu") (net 1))
 (segment (start 136.731774 95.141) (end 145.376 86.496774) (width 0.2) (layer "F.Cu") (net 1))
 (segment (start 89.29 87.67) (end 96.761 95.141) (width 0.2) (layer "F.Cu") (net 1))
 (segment (start 96.761 95.141) (end 136.731774 95.141) (width 0.2) (layer "F.Cu") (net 1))
 (segment (start 137 80.25) (end 137 81.5) (width 0.2) (layer "F.Cu") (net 1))
 (segment (start 145.376 80.903226) (end 143.996774 79.524) (width 0.2) (layer "F.Cu") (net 1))
 (segment (start 102.25 70.77) (end 102.19 70.71) (width 0.2) (layer "F.Cu") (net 4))
 (segment (start 102.25 90.25) (end 102.25 70.77) (width 0.2) (layer "F.Cu") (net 4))
 (segment (start 132.278 89.472) (end 136 85.75) (width 0.2) (layer "F.Cu") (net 5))
 (segment (start 139 85.5) (end 139 83.002226) (width 0.2) (layer "F.Cu") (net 5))
 (segment (start 127.293586 89.472) (end 132.278 89.472) (width 0.2) (layer "F.Cu") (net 5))
 (segment (start 108.6 87.71) (end 125.531586 87.71) (width 0.2) (layer "F.Cu") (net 5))
 (segment (start 139 83.002226) (end 138.296774 82.299) (width 0.2) (layer "F.Cu") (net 5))
 (segment (start 125.531586 87.71) (end 127.293586 89.472) (width 0.2) (layer "F.Cu") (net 5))
 (via (at 136 85.75) (size 0.6) (drill 0.3) (layers "F.Cu" "B.Cu") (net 5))
 (via (at 139 85.5) (size 0.6) (drill 0.3) (layers "F.Cu" "B.Cu") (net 5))
 (segment (start 136 85.75) (end 136.25 85.5) (width 0.2) (layer "B.Cu") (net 5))
 (segment (start 136.25 85.5) (end 139 85.5) (width 0.2) (layer "B.Cu") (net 5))
 (segment (start 105.25847 90.21) (end 121.69 90.21) (width 0.2) (layer "F.Cu") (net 53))
 (segment (start 100.48253 93.991) (end 101.47747 93.991) (width 0.2) (layer "F.Cu") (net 53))
 (segment (start 83.52 77.02847) (end 100.48253 93.991) (width 0.2) (layer "F.Cu") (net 53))
 (segment (start 101.47747 93.991) (end 105.25847 90.21) (width 0.2) (layer "F.Cu") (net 53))
 (segment (start 83.52 70.46) (end 83.52 77.02847) (width 0.2) (layer "F.Cu") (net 53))
 (segment (start 132.46 83.25) (end 134.75 83.25) (width 0.2) (layer "F.Cu") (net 8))
 (segment (start 137.060126 83.1) (end 137.7625 83.1) (width 0.2) (layer "F.Cu") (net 8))
 (segment (start 128.04 87.67) (end 132.46 83.25) (width 0.2) (layer "F.Cu") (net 8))
 (segment (start 136.5 83) (end 136.75 83.25) (width 0.2) (layer "F.Cu") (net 8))
 (segment (start 136.75 83.25) (end 136.980063 83.019937) (width 0.2) (layer "F.Cu") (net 8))
 (segment (start 134.75 83.25) (end 135 83) (width 0.2) (layer "F.Cu") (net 8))
 (segment (start 136.980063 83.019937) (end 137.060126 83.1) (width 0.2) (layer "F.Cu") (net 8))
 (segment (start 135 83) (end 136.5 83) (width 0.2) (layer "F.Cu") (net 8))
 (segment (start 108.219 86.269) (end 124.657686 86.269) (width 0.2) (layer "F.Cu") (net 9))
 (segment (start 136.915686 83.65) (end 137.065686 83.5) (width 0.2) (layer "F.Cu") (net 9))
 (segment (start 89.87 67.92) (end 89.87 79.851314) (width 0.2) (layer "F.Cu") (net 9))
 (segment (start 103.665685 90.815629) (end 103.665685 87.9) (width 0.2) (layer "F.Cu") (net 9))
 (segment (start 106.665685 84.9) (end 106.85 84.9) (width 0.2) (layer "F.Cu") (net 9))
 (segment (start 101.669686 91.651) (end 102.830314 91.651) (width 0.2) (layer "F.Cu") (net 9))
 (segment (start 103.665685 87.9) (end 106.665685 84.9) (width 0.2) (layer "F.Cu") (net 9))
 (segment (start 131.179 89.071) (end 136.6 83.65) (width 0.2) (layer "F.Cu") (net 9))
 (segment (start 106.85 84.9) (end 108.219 86.269) (width 0.2) (layer "F.Cu") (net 9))
 (segment (start 136.6 83.65) (end 136.915686 83.65) (width 0.2) (layer "F.Cu") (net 9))
 (segment (start 137.065686 83.5) (end 137.7625 83.5) (width 0.2) (layer "F.Cu") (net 9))
 (segment (start 89.87 79.851314) (end 101.669686 91.651) (width 0.2) (layer "F.Cu") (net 9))
 (segment (start 124.657686 86.269) (end 127.459686 89.071) (width 0.2) (layer "F.Cu") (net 9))
 (segment (start 102.830314 91.651) (end 103.665685 90.815629) (width 0.2) (layer "F.Cu") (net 9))
 (segment (start 127.459686 89.071) (end 131.179 89.071) (width 0.2) (layer "F.Cu") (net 9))
 (segment (start 108.54 68.17) (end 109.941 66.769) (width 0.2) (layer "F.Cu") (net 3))
 (segment (start 109.941 66.769) (end 131.241774 66.769) (width 0.2) (layer "F.Cu") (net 3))
 (segment (start 135.75 80.422774) (end 136.6 81.272774) (width 0.2) (layer "F.Cu") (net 3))
 (segment (start 135.75 71.277226) (end 135.75 80.422774) (width 0.2) (layer "F.Cu") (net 3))
 (segment (start 136.834315 81.9) (end 137.7625 81.9) (width 0.2) (layer "F.Cu") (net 3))
 (segment (start 136.6 81.665685) (end 136.834315 81.9) (width 0.2) (layer "F.Cu") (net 3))
 (segment (start 131.241774 66.769) (end 135.75 71.277226) (width 0.2) (layer "F.Cu") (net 3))
 (segment (start 136.6 81.272774) (end 136.6 81.665685) (width 0.2) (layer "F.Cu") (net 3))
 (segment (start 128.12 73.751371) (end 128.12 68.17) (width 0.2) (layer "F.Cu") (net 7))
 (segment (start 136.967629 82.599) (end 128.12 73.751371) (width 0.2) (layer "F.Cu") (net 7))
 (segment (start 137.126226 82.599) (end 137.227226 82.7) (width 0.2) (layer "F.Cu") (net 7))
 (segment (start 137.7625 82.7) (end 137.227226 82.7) (width 0.2) (layer "F.Cu") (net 7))
 (segment (start 137.126226 82.599) (end 136.967629 82.599) (width 0.2) (layer "F.Cu") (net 7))
 (segment (start 144.452226 80.75) (end 143.710672 81.491554) (width 0.2) (layer "F.Cu") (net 6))
 (segment (start 141.4 80.797774) (end 141.702226 81.1) (width 0.2) (layer "F.Cu") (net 6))
 (segment (start 144.6375 81.1) (end 144.5 80.9625) (width 0.2) (layer "F.Cu") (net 6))
 (segment (start 138.35 81.1) (end 139 81.75) (width 0.2) (layer "F.Cu") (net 6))
 (segment (start 144.5 80.9625) (end 144.5 80.75) (width 0.2) (layer "F.Cu") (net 6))
 (segment (start 136.5 84.75) (end 137.177226 84.75) (width 0.2) (layer "F.Cu") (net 6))
 (segment (start 143.75 85.208219) (end 143.708976 85.249243) (width 0.2) (layer "F.Cu") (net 6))
 (segment (start 137.7625 81.1) (end 138.35 81.1) (width 0.2) (layer "F.Cu") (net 6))
 (segment (start 141.702226 81.1) (end 144.6375 81.1) (width 0.2) (layer "F.Cu") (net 6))
 (segment (start 143.75 84.75) (end 143.75 85.208219) (width 0.2) (layer "F.Cu") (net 6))
 (segment (start 144.6375 84.7) (end 143.8 84.7) (width 0.2) (layer "F.Cu") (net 6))
 (segment (start 144.5 80.75) (end 144.452226 80.75) (width 0.2) (layer "F.Cu") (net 6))
 (segment (start 137.177226 84.75) (end 137.227226 84.7) (width 0.2) (layer "F.Cu") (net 6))
 (segment (start 143.8 84.7) (end 143.75 84.75) (width 0.2) (layer "F.Cu") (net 6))
 (segment (start 143.710672 81.491554) (end 143.710672 81.742176) (width 0.2) (layer "F.Cu") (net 6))
 (segment (start 137.7625 84.7) (end 137.227226 84.7) (width 0.2) (layer "F.Cu") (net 6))
 (segment (start 141.4 88.4) (end 141.75 88.75) (width 0.2) (layer "F.Cu") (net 6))
 (segment (start 141.4 87.1375) (end 141.4 88.4) (width 0.2) (layer "F.Cu") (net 6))
 (segment (start 141.4 80.2625) (end 141.4 80.797774) (width 0.2) (layer "F.Cu") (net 6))
 (via (at 141.75 88.75) (size 0.6) (drill 0.3) (layers "F.Cu" "B.Cu") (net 6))
 (via (at 143.708976 85.249243) (size 0.6) (drill 0.3) (layers "F.Cu" "B.Cu") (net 6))
 (via (at 143.710672 81.742176) (size 0.6) (drill 0.3) (layers "F.Cu" "B.Cu") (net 6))
 (via (at 136.5 84.75) (size 0.6) (drill 0.3) (layers "F.Cu" "B.Cu") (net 6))
 (via (at 139 81.75) (size 0.6) (drill 0.3) (layers "F.Cu" "B.Cu") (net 6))
 (segment (start 143.25 88.75) (end 141.75 88.75) (width 0.2) (layer "B.Cu") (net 6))
 (segment (start 143.708976 85.249243) (end 141.75 87.208219) (width 0.2) (layer "B.Cu") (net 6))
 (segment (start 133.75 85.5) (end 134.5 84.75) (width 0.2) (layer "B.Cu") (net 6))
 (segment (start 142.75 81.75) (end 146 85) (width 0.2) (layer "B.Cu") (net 6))
 (segment (start 141.75 87.208219) (end 141.75 88.75) (width 0.2) (layer "B.Cu") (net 6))
 (segment (start 146 86) (end 143.25 88.75) (width 0.2) (layer "B.Cu") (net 6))
 (segment (start 146 85) (end 146 86) (width 0.2) (layer "B.Cu") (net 6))
 (segment (start 135.75 88.75) (end 135.75 87.5) (width 0.2) (layer "B.Cu") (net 6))
 (segment (start 135.75 87.5) (end 133.75 85.5) (width 0.2) (layer "B.Cu") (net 6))
 (segment (start 139 81.75) (end 142.75 81.75) (width 0.2) (layer "B.Cu") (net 6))
 (segment (start 134.5 84.75) (end 136.5 84.75) (width 0.2) (layer "B.Cu") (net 6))
 (segment (start 141.75 88.75) (end 135.75 88.75) (width 0.2) (layer "B.Cu") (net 6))
 (segment (start 142.152226 86.25) (end 141.799 86.603226) (width 0.2) (layer "F.Cu") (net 23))
 (segment (start 141 80.2625) (end 141 81.25) (width 0.2) (layer "F.Cu") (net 23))
 (segment (start 142.452 86.25) (end 142.152226 86.25) (width 0.2) (layer "F.Cu") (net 23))
 (segment (start 141 81.25) (end 141.549 81.799) (width 0.2) (layer "F.Cu") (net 23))
 (segment (start 143.101 85.601) (end 142.452 86.25) (width 0.2) (layer "F.Cu") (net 23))
 (segment (start 141.549 81.799) (end 143.101 81.799) (width 0.2) (layer "F.Cu") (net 23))
 (segment (start 143.101 81.799) (end 143.101 85.601) (width 0.2) (layer "F.Cu") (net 23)))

